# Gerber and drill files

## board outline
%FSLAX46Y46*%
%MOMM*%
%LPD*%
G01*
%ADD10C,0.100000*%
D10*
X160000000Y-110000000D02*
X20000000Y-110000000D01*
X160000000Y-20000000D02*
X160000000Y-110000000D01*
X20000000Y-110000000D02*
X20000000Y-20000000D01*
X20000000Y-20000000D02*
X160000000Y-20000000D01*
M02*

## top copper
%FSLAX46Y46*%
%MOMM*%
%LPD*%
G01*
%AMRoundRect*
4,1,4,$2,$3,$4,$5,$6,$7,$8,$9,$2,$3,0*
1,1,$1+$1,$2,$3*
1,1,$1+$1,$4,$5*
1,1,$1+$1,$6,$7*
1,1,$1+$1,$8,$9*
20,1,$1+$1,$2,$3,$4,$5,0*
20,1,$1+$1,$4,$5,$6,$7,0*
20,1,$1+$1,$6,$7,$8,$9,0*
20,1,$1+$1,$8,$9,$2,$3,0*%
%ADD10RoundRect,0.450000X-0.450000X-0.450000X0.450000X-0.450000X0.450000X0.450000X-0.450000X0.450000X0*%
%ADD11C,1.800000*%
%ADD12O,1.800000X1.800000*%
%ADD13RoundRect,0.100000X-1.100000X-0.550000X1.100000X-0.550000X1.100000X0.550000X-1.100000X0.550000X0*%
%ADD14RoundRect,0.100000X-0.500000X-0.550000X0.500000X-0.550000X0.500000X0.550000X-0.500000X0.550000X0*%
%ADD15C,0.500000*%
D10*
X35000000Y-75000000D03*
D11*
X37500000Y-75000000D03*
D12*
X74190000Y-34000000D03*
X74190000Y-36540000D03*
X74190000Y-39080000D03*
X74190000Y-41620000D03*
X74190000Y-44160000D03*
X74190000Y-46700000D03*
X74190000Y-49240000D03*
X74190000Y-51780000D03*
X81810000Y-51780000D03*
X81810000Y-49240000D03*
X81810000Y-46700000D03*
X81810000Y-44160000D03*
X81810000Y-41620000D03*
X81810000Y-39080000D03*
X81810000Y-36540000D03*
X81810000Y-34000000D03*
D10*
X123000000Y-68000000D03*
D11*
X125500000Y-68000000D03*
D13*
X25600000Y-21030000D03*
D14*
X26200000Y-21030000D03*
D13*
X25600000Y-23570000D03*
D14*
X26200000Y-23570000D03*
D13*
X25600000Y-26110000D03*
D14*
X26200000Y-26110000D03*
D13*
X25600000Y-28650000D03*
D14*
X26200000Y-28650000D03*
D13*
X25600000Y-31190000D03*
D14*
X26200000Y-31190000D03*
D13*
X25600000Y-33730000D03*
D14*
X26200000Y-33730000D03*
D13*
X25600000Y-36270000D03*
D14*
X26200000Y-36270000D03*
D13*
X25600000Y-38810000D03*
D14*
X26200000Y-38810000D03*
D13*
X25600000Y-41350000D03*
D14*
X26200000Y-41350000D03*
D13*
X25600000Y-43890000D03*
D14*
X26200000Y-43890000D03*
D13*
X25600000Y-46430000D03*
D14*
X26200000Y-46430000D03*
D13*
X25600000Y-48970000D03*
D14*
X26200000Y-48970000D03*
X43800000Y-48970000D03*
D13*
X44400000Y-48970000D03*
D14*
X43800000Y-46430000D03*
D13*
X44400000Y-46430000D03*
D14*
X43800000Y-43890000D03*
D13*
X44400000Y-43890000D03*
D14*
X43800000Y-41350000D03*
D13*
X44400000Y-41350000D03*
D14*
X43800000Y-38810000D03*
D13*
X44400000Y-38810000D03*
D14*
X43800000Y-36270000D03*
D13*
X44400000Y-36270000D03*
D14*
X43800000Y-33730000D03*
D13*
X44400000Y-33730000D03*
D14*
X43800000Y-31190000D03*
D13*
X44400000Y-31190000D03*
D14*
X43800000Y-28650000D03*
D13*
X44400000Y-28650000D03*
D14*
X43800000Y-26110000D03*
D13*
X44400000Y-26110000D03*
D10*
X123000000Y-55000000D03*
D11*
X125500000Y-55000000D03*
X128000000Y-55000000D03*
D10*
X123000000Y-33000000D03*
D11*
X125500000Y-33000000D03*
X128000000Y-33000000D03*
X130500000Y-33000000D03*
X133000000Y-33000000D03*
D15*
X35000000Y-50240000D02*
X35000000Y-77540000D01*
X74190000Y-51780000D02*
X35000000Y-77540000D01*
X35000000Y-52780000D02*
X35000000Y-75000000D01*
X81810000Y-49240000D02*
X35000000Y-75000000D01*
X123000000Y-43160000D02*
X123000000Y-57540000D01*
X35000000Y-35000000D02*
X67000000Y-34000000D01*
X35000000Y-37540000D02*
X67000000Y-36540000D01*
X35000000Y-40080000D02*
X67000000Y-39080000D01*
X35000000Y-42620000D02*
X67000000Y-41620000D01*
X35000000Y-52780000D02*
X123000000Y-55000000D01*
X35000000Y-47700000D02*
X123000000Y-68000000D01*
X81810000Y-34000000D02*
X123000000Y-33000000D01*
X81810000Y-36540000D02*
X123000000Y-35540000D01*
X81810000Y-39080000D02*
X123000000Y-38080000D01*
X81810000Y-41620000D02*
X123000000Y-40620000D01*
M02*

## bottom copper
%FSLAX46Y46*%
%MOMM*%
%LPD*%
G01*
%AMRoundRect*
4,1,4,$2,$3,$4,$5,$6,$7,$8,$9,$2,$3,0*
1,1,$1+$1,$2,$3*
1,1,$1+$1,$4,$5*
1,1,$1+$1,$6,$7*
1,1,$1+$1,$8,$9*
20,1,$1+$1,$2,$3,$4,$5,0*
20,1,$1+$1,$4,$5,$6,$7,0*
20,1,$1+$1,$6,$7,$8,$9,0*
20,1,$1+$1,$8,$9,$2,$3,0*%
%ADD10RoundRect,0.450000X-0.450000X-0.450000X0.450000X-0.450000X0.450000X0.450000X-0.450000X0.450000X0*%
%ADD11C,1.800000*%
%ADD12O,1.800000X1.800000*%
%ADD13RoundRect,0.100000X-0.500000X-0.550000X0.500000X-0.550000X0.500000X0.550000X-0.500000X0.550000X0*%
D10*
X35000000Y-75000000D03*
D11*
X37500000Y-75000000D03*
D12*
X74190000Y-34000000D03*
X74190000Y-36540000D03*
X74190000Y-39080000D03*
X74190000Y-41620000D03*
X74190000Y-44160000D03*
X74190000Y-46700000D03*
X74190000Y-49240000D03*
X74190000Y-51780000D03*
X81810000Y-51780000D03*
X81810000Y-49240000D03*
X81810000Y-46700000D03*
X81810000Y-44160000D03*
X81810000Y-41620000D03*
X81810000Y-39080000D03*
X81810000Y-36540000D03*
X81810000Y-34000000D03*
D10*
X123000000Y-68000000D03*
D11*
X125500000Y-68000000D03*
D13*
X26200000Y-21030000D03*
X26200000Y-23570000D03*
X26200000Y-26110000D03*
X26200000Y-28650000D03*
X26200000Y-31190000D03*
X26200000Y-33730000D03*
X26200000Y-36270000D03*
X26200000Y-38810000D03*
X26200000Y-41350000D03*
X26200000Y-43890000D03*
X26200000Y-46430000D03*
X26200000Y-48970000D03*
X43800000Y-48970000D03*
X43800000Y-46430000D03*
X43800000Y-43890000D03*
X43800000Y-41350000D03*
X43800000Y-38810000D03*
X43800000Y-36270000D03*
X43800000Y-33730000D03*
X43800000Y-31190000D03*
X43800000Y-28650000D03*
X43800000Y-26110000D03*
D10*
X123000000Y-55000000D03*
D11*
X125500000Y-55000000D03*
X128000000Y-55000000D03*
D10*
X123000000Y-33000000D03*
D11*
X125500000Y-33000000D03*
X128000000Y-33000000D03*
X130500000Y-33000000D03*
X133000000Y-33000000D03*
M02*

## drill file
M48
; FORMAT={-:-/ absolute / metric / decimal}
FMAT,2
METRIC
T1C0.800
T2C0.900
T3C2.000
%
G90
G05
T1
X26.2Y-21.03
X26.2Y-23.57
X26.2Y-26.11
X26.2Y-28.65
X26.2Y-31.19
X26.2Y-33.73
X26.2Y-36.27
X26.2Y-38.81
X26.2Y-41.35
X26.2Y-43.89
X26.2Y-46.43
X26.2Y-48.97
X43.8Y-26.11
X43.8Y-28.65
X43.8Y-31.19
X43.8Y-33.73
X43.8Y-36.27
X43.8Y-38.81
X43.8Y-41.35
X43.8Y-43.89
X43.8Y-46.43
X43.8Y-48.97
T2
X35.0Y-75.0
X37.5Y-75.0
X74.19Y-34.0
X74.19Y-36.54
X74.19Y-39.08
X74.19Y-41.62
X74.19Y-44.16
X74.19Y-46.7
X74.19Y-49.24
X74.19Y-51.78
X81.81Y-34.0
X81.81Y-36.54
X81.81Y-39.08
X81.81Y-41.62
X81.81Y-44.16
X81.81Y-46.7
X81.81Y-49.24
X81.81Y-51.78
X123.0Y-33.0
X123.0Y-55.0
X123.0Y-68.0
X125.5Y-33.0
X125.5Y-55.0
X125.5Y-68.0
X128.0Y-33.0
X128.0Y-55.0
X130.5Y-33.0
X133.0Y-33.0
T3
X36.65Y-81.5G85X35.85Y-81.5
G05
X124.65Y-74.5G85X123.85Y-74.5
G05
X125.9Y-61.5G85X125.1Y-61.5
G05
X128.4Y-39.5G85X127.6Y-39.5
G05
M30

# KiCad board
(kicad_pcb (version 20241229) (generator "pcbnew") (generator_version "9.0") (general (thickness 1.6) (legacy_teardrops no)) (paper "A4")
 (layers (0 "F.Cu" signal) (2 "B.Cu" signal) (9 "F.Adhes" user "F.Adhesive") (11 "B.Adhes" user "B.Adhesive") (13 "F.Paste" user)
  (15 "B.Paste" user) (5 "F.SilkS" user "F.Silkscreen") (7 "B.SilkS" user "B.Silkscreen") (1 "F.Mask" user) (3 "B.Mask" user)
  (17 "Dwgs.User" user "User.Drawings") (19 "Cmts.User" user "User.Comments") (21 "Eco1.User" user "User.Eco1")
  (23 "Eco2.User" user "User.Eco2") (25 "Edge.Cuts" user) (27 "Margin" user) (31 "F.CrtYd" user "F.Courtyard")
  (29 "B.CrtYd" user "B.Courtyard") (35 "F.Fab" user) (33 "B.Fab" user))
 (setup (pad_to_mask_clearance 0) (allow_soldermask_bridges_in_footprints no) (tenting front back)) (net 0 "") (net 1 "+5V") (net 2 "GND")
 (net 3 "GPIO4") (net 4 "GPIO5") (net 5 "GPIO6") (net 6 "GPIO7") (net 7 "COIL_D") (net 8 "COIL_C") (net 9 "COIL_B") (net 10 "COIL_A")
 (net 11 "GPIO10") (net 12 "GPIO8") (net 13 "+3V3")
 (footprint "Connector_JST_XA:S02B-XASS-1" (layer "F.Cu") (at 35 75)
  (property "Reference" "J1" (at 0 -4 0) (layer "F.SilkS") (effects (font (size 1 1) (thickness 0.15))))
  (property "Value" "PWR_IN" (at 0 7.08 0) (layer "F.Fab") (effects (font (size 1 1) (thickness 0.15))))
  (pad "" np_thru_hole oval (at 1.25 6.5 180) (size 2.8 2) (drill oval 2.8 2) (layers "*.Cu" "*.Mask"))
  (pad "1" thru_hole roundrect (at 0 0) (size 1.8 1.8) (drill 0.9) (layers "*.Cu" "*.Mask") (remove_unused_layers no)
   (roundrect_rratio 0.25) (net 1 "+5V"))
  (pad "2" thru_hole circle (at 2.5 0) (size 1.8 1.8) (drill 0.9) (layers "*.Cu" "*.Mask") (remove_unused_layers no) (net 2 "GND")))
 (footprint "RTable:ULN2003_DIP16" (layer "F.Cu") (at 78 34)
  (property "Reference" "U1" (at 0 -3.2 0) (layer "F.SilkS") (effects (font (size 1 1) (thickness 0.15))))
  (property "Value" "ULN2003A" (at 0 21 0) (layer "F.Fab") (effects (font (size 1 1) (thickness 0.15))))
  (pad "1" thru_hole oval (at -3.81 0) (size 1.8 1.8) (drill 0.9) (layers "*.Cu" "*.Mask") (remove_unused_layers no) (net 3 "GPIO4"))
  (pad "2" thru_hole oval (at -3.81 2.54) (size 1.8 1.8) (drill 0.9) (layers "*.Cu" "*.Mask") (remove_unused_layers no) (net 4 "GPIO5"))
  (pad "3" thru_hole oval (at -3.81 5.08) (size 1.8 1.8) (drill 0.9) (layers "*.Cu" "*.Mask") (remove_unused_layers no) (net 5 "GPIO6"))
  (pad "4" thru_hole oval (at -3.81 7.62) (size 1.8 1.8) (drill 0.9) (layers "*.Cu" "*.Mask") (remove_unused_layers no) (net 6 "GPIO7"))
  (pad "5" thru_hole oval (at -3.81 10.16) (size 1.8 1.8) (drill 0.9) (layers "*.Cu" "*.Mask") (remove_unused_layers no))
  (pad "6" thru_hole oval (at -3.81 12.7) (size 1.8 1.8) (drill 0.9) (layers "*.Cu" "*.Mask") (remove_unused_layers no))
  (pad "7" thru_hole oval (at -3.81 15.24) (size 1.8 1.8) (drill 0.9) (layers "*.Cu" "*.Mask") (remove_unused_layers no))
  (pad "8" thru_hole oval (at -3.81 17.78) (size 1.8 1.8) (drill 0.9) (layers "*.Cu" "*.Mask") (remove_unused_layers no) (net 2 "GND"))
  (pad "9" thru_hole oval (at 3.81 17.78) (size 1.8 1.8) (drill 0.9) (layers "*.Cu" "*.Mask") (remove_unused_layers no) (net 1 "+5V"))
  (pad "10" thru_hole oval (at 3.81 15.24) (size 1.8 1.8) (drill 0.9) (layers "*.Cu" "*.Mask") (remove_unused_layers no))
  (pad "11" thru_hole oval (at 3.81 12.7) (size 1.8 1.8) (drill 0.9) (layers "*.Cu" "*.Mask") (remove_unused_layers no))
  (pad "12" thru_hole oval (at 3.81 10.16) (size 1.8 1.8) (drill 0.9) (layers "*.Cu" "*.Mask") (remove_unused_layers no))
  (pad "13" thru_hole oval (at 3.81 7.62) (size 1.8 1.8) (drill 0.9) (layers "*.Cu" "*.Mask") (remove_unused_layers no) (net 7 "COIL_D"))
  (pad "14" thru_hole oval (at 3.81 5.08) (size 1.8 1.8) (drill 0.9) (layers "*.Cu" "*.Mask") (remove_unused_layers no) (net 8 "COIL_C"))
  (pad "15" thru_hole oval (at 3.81 2.54) (size 1.8 1.8) (drill 0.9) (layers "*.Cu" "*.Mask") (remove_unused_layers no) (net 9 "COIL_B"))
  (pad "16" thru_hole oval (at 3.81 0) (size 1.8 1.8) (drill 0.9) (layers "*.Cu" "*.Mask") (remove_unused_layers no) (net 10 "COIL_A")))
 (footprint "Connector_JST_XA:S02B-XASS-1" (layer "F.Cu") (at 123 68)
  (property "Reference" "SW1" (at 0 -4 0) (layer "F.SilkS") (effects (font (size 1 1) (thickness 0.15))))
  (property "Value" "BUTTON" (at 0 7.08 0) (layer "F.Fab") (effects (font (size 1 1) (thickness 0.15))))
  (pad "" np_thru_hole oval (at 1.25 6.5 180) (size 2.8 2) (drill oval 2.8 2) (layers "*.Cu" "*.Mask"))
  (pad "1" thru_hole roundrect (at 0 0) (size 1.8 1.8) (drill 0.9) (layers "*.Cu" "*.Mask") (remove_unused_layers no)
   (roundrect_rratio 0.25) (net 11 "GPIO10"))
  (pad "2" thru_hole circle (at 2.5 0) (size 1.8 1.8) (drill 0.9) (layers "*.Cu" "*.Mask") (remove_unused_layers no) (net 2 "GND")))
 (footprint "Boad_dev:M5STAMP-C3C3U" (layer "F.Cu") (at 35 35)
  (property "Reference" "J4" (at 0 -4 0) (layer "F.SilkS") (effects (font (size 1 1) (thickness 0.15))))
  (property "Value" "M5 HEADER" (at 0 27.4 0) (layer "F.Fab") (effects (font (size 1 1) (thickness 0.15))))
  (pad "1" smd roundrect (at -9.4 -13.97) (size 2.4 1.3) (layers "F.Cu" "F.Mask" "F.Paste") (roundrect_rratio 0.07692307692) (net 3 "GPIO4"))
  (pad "1" thru_hole roundrect (at -8.8 -13.97) (size 1.2 1.3) (drill 0.8) (layers "*.Cu" "*.Mask") (remove_unused_layers no)
   (roundrect_rratio 0.08333333333) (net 3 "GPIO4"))
  (pad "2" smd roundrect (at -9.4 -11.43) (size 2.4 1.3) (layers "F.Cu" "F.Mask" "F.Paste") (roundrect_rratio 0.07692307692) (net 4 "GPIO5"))
  (pad "2" thru_hole roundrect (at -8.8 -11.43) (size 1.2 1.3) (drill 0.8) (layers "*.Cu" "*.Mask") (remove_unused_layers no)
   (roundrect_rratio 0.08333333333) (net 4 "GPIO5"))
  (pad "3" smd roundrect (at -9.4 -8.89) (size 2.4 1.3) (layers "F.Cu" "F.Mask" "F.Paste") (roundrect_rratio 0.07692307692) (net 5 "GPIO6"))
  (pad "3" thru_hole roundrect (at -8.8 -8.89) (size 1.2 1.3) (drill 0.8) (layers "*.Cu" "*.Mask") (remove_unused_layers no)
   (roundrect_rratio 0.08333333333) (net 5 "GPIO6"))
  (pad "4" smd roundrect (at -9.4 -6.35) (size 2.4 1.3) (layers "F.Cu" "F.Mask" "F.Paste") (roundrect_rratio 0.07692307692) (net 6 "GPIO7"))
  (pad "4" thru_hole roundrect (at -8.8 -6.35) (size 1.2 1.3) (drill 0.8) (layers "*.Cu" "*.Mask") (remove_unused_layers no)
   (roundrect_rratio 0.08333333333) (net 6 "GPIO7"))
  (pad "5" smd roundrect (at -9.4 -3.81) (size 2.4 1.3) (layers "F.Cu" "F.Mask" "F.Paste") (roundrect_rratio 0.07692307692) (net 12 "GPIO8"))
  (pad "5" thru_hole roundrect (at -8.8 -3.81) (size 1.2 1.3) (drill 0.8) (layers "*.Cu" "*.Mask") (remove_unused_layers no)
   (roundrect_rratio 0.08333333333) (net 12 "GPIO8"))
  (pad "6" smd roundrect (at -9.4 -1.27) (size 2.4 1.3) (layers "F.Cu" "F.Mask" "F.Paste") (roundrect_rratio 0.07692307692)
   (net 11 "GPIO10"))
  (pad "6" thru_hole roundrect (at -8.8 -1.27) (size 1.2 1.3) (drill 0.8) (layers "*.Cu" "*.Mask") (remove_unused_layers no)
   (roundrect_rratio 0.08333333333) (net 11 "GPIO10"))
  (pad "7" smd roundrect (at -9.4 1.27) (size 2.4 1.3) (layers "F.Cu" "F.Mask" "F.Paste") (roundrect_rratio 0.07692307692) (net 2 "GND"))
  (pad "7" thru_hole roundrect (at -8.8 1.27) (size 1.2 1.3) (drill 0.8) (layers "*.Cu" "*.Mask") (remove_unused_layers no)
   (roundrect_rratio 0.08333333333) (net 2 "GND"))
  (pad "8" smd roundrect (at -9.4 3.81) (size 2.4 1.3) (layers "F.Cu" "F.Mask" "F.Paste") (roundrect_rratio 0.07692307692) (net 1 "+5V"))
  (pad "8" thru_hole roundrect (at -8.8 3.81) (size 1.2 1.3) (drill 0.8) (layers "*.Cu" "*.Mask") (remove_unused_layers no)
   (roundrect_rratio 0.08333333333) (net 1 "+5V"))
  (pad "9" smd roundrect (at -9.4 6.35) (size 2.4 1.3) (layers "F.Cu" "F.Mask" "F.Paste") (roundrect_rratio 0.07692307692) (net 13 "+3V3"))
  (pad "9" thru_hole roundrect (at -8.8 6.35) (size 1.2 1.3) (drill 0.8) (layers "*.Cu" "*.Mask") (remove_unused_layers no)
   (roundrect_rratio 0.08333333333) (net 13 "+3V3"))
  (pad "10" smd roundrect (at -9.4 8.89) (size 2.4 1.3) (layers "F.Cu" "F.Mask" "F.Paste") (roundrect_rratio 0.07692307692))
  (pad "10" thru_hole roundrect (at -8.8 8.89) (size 1.2 1.3) (drill 0.8) (layers "*.Cu" "*.Mask") (remove_unused_layers no)
   (roundrect_rratio 0.08333333333))
  (pad "11" smd roundrect (at -9.4 11.43) (size 2.4 1.3) (layers "F.Cu" "F.Mask" "F.Paste") (roundrect_rratio 0.07692307692))
  (pad "11" thru_hole roundrect (at -8.8 11.43) (size 1.2 1.3) (drill 0.8) (layers "*.Cu" "*.Mask") (remove_unused_layers no)
   (roundrect_rratio 0.08333333333))
  (pad "12" smd roundrect (at -9.4 13.97) (size 2.4 1.3) (layers "F.Cu" "F.Mask" "F.Paste") (roundrect_rratio 0.07692307692))
  (pad "12" thru_hole roundrect (at -8.8 13.97) (size 1.2 1.3) (drill 0.8) (layers "*.Cu" "*.Mask") (remove_unused_layers no)
   (roundrect_rratio 0.08333333333))
  (pad "13" thru_hole roundrect (at 8.8 13.97) (size 1.2 1.3) (drill 0.8) (layers "*.Cu" "*.Mask") (remove_unused_layers no)
   (roundrect_rratio 0.08333333333))
  (pad "13" smd roundrect (at 9.4 13.97) (size 2.4 1.3) (layers "F.Cu" "F.Mask" "F.Paste") (roundrect_rratio 0.07692307692))
  (pad "14" thru_hole roundrect (at 8.8 11.43) (size 1.2 1.3) (drill 0.8) (layers "*.Cu" "*.Mask") (remove_unused_layers no)
   (roundrect_rratio 0.08333333333))
  (pad "14" smd roundrect (at 9.4 11.43) (size 2.4 1.3) (layers "F.Cu" "F.Mask" "F.Paste") (roundrect_rratio 0.07692307692))
  (pad "15" thru_hole roundrect (at 8.8 8.89) (size 1.2 1.3) (drill 0.8) (layers "*.Cu" "*.Mask") (remove_unused_layers no)
   (roundrect_rratio 0.08333333333))
  (pad "15" smd roundrect (at 9.4 8.89) (size 2.4 1.3) (layers "F.Cu" "F.Mask" "F.Paste") (roundrect_rratio 0.07692307692))
  (pad "16" thru_hole roundrect (at 8.8 6.35) (size 1.2 1.3) (drill 0.8) (layers "*.Cu" "*.Mask") (remove_unused_layers no)
   (roundrect_rratio 0.08333333333))
  (pad "16" smd roundrect (at 9.4 6.35) (size 2.4 1.3) (layers "F.Cu" "F.Mask" "F.Paste") (roundrect_rratio 0.07692307692))
  (pad "17" thru_hole roundrect (at 8.8 3.81) (size 1.2 1.3) (drill 0.8) (layers "*.Cu" "*.Mask") (remove_unused_layers no)
   (roundrect_rratio 0.08333333333))
  (pad "17" smd roundrect (at 9.4 3.81) (size 2.4 1.3) (layers "F.Cu" "F.Mask" "F.Paste") (roundrect_rratio 0.07692307692))
  (pad "18" thru_hole roundrect (at 8.8 1.27) (size 1.2 1.3) (drill 0.8) (layers "*.Cu" "*.Mask") (remove_unused_layers no)
   (roundrect_rratio 0.08333333333))
  (pad "18" smd roundrect (at 9.4 1.27) (size 2.4 1.3) (layers "F.Cu" "F.Mask" "F.Paste") (roundrect_rratio 0.07692307692))
  (pad "19" thru_hole roundrect (at 8.8 -1.27) (size 1.2 1.3) (drill 0.8) (layers "*.Cu" "*.Mask") (remove_unused_layers no)
   (roundrect_rratio 0.08333333333))
  (pad "19" smd roundrect (at 9.4 -1.27) (size 2.4 1.3) (layers "F.Cu" "F.Mask" "F.Paste") (roundrect_rratio 0.07692307692))
  (pad "20" thru_hole roundrect (at 8.8 -3.81) (size 1.2 1.3) (drill 0.8) (layers "*.Cu" "*.Mask") (remove_unused_layers no)
   (roundrect_rratio 0.08333333333))
  (pad "20" smd roundrect (at 9.4 -3.81) (size 2.4 1.3) (layers "F.Cu" "F.Mask" "F.Paste") (roundrect_rratio 0.07692307692))
  (pad "21" thru_hole roundrect (at 8.8 -6.35) (size 1.2 1.3) (drill 0.8) (layers "*.Cu" "*.Mask") (remove_unused_layers no)
   (roundrect_rratio 0.08333333333))
  (pad "21" smd roundrect (at 9.4 -6.35) (size 2.4 1.3) (layers "F.Cu" "F.Mask" "F.Paste") (roundrect_rratio 0.07692307692))
  (pad "22" thru_hole roundrect (at 8.8 -8.89) (size 1.2 1.3) (drill 0.8) (layers "*.Cu" "*.Mask") (remove_unused_layers no)
   (roundrect_rratio 0.08333333333))
  (pad "22" smd roundrect (at 9.4 -8.89) (size 2.4 1.3) (layers "F.Cu" "F.Mask" "F.Paste") (roundrect_rratio 0.07692307692)))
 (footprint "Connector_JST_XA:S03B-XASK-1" (layer "F.Cu") (at 123 55)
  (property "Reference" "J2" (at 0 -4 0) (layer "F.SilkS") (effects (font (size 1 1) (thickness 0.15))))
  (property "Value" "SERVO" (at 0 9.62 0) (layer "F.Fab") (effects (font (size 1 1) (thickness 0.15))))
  (pad "" np_thru_hole oval (at 2.5 6.5 180) (size 2.8 2) (drill oval 2.8 2) (layers "*.Cu" "*.Mask"))
  (pad "1" thru_hole roundrect (at 0 0) (size 1.8 1.8) (drill 0.9) (layers "*.Cu" "*.Mask") (remove_unused_layers no)
   (roundrect_rratio 0.25) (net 12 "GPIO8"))
  (pad "2" thru_hole circle (at 2.5 0) (size 1.8 1.8) (drill 0.9) (layers "*.Cu" "*.Mask") (remove_unused_layers no) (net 1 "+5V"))
  (pad "3" thru_hole circle (at 5 0) (size 1.8 1.8) (drill 0.9) (layers "*.Cu" "*.Mask") (remove_unused_layers no) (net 2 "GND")))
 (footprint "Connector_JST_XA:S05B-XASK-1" (layer "F.Cu") (at 123 33)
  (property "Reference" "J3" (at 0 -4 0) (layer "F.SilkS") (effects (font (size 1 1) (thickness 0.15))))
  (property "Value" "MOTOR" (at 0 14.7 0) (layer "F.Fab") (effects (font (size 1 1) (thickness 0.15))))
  (pad "" np_thru_hole oval (at 5 6.5 180) (size 2.8 2) (drill oval 2.8 2) (layers "*.Cu" "*.Mask"))
  (pad "1" thru_hole roundrect (at 0 0) (size 1.8 1.8) (drill 0.9) (layers "*.Cu" "*.Mask") (remove_unused_layers no)
   (roundrect_rratio 0.25) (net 10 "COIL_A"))
  (pad "2" thru_hole circle (at 2.5 0) (size 1.8 1.8) (drill 0.9) (layers "*.Cu" "*.Mask") (remove_unused_layers no) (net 9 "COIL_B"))
  (pad "3" thru_hole circle (at 5 0) (size 1.8 1.8) (drill 0.9) (layers "*.Cu" "*.Mask") (remove_unused_layers no) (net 8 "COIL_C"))
  (pad "4" thru_hole circle (at 7.5 0) (size 1.8 1.8) (drill 0.9) (layers "*.Cu" "*.Mask") (remove_unused_layers no) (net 7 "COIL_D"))
  (pad "5" thru_hole circle (at 10 0) (size 1.8 1.8) (drill 0.9) (layers "*.Cu" "*.Mask") (remove_unused_layers no) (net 1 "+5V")))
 (gr_line (start 160 110) (end 20 110) (stroke (width 0.1) (type default)) (layer "Edge.Cuts"))
 (gr_line (start 160 20) (end 160 110) (stroke (width 0.1) (type default)) (layer "Edge.Cuts"))
 (gr_line (start 20 110) (end 20 20) (stroke (width 0.1) (type default)) (layer "Edge.Cuts"))
 (gr_line (start 20 20) (end 160 20) (stroke (width 0.1) (type default)) (layer "Edge.Cuts"))
 (segment (start 35 50.24) (end 35 77.54) (width 0.5) (layer "F.Cu") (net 2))
 (segment (start 74.19 51.78) (end 35 77.54) (width 0.5) (layer "F.Cu") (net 2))
 (segment (start 35 52.78) (end 35 75) (width 0.5) (layer "F.Cu") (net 1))
 (segment (start 81.81 49.24) (end 35 75) (width 0.5) (layer "F.Cu") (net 1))
 (segment (start 123 43.16) (end 123 57.54) (width 0.5) (layer "F.Cu") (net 1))
 (segment (start 35 35) (end 67 34) (width 0.5) (layer "F.Cu") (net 3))
 (segment (start 35 37.54) (end 67 36.54) (width 0.5) (layer "F.Cu") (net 4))
 (segment (start 35 40.08) (end 67 39.08) (width 0.5) (layer "F.Cu") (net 5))
 (segment (start 35 42.62) (end 67 41.62) (width 0.5) (layer "F.Cu") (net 6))
 (segment (start 35 52.78) (end 123 55) (width 0.5) (layer "F.Cu") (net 12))
 (segment (start 35 47.7) (end 123 68) (width 0.5) (layer "F.Cu") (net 11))
 (segment (start 81.81 34) (end 123 33) (width 0.5) (layer "F.Cu") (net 10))
 (segment (start 81.81 36.54) (end 123 35.54) (width 0.5) (layer "F.Cu") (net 9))
 (segment (start 81.81 39.08) (end 123 38.08) (width 0.5) (layer "F.Cu") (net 8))
 (segment (start 81.81 41.62) (end 123 40.62) (width 0.5) (layer "F.Cu") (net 7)))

